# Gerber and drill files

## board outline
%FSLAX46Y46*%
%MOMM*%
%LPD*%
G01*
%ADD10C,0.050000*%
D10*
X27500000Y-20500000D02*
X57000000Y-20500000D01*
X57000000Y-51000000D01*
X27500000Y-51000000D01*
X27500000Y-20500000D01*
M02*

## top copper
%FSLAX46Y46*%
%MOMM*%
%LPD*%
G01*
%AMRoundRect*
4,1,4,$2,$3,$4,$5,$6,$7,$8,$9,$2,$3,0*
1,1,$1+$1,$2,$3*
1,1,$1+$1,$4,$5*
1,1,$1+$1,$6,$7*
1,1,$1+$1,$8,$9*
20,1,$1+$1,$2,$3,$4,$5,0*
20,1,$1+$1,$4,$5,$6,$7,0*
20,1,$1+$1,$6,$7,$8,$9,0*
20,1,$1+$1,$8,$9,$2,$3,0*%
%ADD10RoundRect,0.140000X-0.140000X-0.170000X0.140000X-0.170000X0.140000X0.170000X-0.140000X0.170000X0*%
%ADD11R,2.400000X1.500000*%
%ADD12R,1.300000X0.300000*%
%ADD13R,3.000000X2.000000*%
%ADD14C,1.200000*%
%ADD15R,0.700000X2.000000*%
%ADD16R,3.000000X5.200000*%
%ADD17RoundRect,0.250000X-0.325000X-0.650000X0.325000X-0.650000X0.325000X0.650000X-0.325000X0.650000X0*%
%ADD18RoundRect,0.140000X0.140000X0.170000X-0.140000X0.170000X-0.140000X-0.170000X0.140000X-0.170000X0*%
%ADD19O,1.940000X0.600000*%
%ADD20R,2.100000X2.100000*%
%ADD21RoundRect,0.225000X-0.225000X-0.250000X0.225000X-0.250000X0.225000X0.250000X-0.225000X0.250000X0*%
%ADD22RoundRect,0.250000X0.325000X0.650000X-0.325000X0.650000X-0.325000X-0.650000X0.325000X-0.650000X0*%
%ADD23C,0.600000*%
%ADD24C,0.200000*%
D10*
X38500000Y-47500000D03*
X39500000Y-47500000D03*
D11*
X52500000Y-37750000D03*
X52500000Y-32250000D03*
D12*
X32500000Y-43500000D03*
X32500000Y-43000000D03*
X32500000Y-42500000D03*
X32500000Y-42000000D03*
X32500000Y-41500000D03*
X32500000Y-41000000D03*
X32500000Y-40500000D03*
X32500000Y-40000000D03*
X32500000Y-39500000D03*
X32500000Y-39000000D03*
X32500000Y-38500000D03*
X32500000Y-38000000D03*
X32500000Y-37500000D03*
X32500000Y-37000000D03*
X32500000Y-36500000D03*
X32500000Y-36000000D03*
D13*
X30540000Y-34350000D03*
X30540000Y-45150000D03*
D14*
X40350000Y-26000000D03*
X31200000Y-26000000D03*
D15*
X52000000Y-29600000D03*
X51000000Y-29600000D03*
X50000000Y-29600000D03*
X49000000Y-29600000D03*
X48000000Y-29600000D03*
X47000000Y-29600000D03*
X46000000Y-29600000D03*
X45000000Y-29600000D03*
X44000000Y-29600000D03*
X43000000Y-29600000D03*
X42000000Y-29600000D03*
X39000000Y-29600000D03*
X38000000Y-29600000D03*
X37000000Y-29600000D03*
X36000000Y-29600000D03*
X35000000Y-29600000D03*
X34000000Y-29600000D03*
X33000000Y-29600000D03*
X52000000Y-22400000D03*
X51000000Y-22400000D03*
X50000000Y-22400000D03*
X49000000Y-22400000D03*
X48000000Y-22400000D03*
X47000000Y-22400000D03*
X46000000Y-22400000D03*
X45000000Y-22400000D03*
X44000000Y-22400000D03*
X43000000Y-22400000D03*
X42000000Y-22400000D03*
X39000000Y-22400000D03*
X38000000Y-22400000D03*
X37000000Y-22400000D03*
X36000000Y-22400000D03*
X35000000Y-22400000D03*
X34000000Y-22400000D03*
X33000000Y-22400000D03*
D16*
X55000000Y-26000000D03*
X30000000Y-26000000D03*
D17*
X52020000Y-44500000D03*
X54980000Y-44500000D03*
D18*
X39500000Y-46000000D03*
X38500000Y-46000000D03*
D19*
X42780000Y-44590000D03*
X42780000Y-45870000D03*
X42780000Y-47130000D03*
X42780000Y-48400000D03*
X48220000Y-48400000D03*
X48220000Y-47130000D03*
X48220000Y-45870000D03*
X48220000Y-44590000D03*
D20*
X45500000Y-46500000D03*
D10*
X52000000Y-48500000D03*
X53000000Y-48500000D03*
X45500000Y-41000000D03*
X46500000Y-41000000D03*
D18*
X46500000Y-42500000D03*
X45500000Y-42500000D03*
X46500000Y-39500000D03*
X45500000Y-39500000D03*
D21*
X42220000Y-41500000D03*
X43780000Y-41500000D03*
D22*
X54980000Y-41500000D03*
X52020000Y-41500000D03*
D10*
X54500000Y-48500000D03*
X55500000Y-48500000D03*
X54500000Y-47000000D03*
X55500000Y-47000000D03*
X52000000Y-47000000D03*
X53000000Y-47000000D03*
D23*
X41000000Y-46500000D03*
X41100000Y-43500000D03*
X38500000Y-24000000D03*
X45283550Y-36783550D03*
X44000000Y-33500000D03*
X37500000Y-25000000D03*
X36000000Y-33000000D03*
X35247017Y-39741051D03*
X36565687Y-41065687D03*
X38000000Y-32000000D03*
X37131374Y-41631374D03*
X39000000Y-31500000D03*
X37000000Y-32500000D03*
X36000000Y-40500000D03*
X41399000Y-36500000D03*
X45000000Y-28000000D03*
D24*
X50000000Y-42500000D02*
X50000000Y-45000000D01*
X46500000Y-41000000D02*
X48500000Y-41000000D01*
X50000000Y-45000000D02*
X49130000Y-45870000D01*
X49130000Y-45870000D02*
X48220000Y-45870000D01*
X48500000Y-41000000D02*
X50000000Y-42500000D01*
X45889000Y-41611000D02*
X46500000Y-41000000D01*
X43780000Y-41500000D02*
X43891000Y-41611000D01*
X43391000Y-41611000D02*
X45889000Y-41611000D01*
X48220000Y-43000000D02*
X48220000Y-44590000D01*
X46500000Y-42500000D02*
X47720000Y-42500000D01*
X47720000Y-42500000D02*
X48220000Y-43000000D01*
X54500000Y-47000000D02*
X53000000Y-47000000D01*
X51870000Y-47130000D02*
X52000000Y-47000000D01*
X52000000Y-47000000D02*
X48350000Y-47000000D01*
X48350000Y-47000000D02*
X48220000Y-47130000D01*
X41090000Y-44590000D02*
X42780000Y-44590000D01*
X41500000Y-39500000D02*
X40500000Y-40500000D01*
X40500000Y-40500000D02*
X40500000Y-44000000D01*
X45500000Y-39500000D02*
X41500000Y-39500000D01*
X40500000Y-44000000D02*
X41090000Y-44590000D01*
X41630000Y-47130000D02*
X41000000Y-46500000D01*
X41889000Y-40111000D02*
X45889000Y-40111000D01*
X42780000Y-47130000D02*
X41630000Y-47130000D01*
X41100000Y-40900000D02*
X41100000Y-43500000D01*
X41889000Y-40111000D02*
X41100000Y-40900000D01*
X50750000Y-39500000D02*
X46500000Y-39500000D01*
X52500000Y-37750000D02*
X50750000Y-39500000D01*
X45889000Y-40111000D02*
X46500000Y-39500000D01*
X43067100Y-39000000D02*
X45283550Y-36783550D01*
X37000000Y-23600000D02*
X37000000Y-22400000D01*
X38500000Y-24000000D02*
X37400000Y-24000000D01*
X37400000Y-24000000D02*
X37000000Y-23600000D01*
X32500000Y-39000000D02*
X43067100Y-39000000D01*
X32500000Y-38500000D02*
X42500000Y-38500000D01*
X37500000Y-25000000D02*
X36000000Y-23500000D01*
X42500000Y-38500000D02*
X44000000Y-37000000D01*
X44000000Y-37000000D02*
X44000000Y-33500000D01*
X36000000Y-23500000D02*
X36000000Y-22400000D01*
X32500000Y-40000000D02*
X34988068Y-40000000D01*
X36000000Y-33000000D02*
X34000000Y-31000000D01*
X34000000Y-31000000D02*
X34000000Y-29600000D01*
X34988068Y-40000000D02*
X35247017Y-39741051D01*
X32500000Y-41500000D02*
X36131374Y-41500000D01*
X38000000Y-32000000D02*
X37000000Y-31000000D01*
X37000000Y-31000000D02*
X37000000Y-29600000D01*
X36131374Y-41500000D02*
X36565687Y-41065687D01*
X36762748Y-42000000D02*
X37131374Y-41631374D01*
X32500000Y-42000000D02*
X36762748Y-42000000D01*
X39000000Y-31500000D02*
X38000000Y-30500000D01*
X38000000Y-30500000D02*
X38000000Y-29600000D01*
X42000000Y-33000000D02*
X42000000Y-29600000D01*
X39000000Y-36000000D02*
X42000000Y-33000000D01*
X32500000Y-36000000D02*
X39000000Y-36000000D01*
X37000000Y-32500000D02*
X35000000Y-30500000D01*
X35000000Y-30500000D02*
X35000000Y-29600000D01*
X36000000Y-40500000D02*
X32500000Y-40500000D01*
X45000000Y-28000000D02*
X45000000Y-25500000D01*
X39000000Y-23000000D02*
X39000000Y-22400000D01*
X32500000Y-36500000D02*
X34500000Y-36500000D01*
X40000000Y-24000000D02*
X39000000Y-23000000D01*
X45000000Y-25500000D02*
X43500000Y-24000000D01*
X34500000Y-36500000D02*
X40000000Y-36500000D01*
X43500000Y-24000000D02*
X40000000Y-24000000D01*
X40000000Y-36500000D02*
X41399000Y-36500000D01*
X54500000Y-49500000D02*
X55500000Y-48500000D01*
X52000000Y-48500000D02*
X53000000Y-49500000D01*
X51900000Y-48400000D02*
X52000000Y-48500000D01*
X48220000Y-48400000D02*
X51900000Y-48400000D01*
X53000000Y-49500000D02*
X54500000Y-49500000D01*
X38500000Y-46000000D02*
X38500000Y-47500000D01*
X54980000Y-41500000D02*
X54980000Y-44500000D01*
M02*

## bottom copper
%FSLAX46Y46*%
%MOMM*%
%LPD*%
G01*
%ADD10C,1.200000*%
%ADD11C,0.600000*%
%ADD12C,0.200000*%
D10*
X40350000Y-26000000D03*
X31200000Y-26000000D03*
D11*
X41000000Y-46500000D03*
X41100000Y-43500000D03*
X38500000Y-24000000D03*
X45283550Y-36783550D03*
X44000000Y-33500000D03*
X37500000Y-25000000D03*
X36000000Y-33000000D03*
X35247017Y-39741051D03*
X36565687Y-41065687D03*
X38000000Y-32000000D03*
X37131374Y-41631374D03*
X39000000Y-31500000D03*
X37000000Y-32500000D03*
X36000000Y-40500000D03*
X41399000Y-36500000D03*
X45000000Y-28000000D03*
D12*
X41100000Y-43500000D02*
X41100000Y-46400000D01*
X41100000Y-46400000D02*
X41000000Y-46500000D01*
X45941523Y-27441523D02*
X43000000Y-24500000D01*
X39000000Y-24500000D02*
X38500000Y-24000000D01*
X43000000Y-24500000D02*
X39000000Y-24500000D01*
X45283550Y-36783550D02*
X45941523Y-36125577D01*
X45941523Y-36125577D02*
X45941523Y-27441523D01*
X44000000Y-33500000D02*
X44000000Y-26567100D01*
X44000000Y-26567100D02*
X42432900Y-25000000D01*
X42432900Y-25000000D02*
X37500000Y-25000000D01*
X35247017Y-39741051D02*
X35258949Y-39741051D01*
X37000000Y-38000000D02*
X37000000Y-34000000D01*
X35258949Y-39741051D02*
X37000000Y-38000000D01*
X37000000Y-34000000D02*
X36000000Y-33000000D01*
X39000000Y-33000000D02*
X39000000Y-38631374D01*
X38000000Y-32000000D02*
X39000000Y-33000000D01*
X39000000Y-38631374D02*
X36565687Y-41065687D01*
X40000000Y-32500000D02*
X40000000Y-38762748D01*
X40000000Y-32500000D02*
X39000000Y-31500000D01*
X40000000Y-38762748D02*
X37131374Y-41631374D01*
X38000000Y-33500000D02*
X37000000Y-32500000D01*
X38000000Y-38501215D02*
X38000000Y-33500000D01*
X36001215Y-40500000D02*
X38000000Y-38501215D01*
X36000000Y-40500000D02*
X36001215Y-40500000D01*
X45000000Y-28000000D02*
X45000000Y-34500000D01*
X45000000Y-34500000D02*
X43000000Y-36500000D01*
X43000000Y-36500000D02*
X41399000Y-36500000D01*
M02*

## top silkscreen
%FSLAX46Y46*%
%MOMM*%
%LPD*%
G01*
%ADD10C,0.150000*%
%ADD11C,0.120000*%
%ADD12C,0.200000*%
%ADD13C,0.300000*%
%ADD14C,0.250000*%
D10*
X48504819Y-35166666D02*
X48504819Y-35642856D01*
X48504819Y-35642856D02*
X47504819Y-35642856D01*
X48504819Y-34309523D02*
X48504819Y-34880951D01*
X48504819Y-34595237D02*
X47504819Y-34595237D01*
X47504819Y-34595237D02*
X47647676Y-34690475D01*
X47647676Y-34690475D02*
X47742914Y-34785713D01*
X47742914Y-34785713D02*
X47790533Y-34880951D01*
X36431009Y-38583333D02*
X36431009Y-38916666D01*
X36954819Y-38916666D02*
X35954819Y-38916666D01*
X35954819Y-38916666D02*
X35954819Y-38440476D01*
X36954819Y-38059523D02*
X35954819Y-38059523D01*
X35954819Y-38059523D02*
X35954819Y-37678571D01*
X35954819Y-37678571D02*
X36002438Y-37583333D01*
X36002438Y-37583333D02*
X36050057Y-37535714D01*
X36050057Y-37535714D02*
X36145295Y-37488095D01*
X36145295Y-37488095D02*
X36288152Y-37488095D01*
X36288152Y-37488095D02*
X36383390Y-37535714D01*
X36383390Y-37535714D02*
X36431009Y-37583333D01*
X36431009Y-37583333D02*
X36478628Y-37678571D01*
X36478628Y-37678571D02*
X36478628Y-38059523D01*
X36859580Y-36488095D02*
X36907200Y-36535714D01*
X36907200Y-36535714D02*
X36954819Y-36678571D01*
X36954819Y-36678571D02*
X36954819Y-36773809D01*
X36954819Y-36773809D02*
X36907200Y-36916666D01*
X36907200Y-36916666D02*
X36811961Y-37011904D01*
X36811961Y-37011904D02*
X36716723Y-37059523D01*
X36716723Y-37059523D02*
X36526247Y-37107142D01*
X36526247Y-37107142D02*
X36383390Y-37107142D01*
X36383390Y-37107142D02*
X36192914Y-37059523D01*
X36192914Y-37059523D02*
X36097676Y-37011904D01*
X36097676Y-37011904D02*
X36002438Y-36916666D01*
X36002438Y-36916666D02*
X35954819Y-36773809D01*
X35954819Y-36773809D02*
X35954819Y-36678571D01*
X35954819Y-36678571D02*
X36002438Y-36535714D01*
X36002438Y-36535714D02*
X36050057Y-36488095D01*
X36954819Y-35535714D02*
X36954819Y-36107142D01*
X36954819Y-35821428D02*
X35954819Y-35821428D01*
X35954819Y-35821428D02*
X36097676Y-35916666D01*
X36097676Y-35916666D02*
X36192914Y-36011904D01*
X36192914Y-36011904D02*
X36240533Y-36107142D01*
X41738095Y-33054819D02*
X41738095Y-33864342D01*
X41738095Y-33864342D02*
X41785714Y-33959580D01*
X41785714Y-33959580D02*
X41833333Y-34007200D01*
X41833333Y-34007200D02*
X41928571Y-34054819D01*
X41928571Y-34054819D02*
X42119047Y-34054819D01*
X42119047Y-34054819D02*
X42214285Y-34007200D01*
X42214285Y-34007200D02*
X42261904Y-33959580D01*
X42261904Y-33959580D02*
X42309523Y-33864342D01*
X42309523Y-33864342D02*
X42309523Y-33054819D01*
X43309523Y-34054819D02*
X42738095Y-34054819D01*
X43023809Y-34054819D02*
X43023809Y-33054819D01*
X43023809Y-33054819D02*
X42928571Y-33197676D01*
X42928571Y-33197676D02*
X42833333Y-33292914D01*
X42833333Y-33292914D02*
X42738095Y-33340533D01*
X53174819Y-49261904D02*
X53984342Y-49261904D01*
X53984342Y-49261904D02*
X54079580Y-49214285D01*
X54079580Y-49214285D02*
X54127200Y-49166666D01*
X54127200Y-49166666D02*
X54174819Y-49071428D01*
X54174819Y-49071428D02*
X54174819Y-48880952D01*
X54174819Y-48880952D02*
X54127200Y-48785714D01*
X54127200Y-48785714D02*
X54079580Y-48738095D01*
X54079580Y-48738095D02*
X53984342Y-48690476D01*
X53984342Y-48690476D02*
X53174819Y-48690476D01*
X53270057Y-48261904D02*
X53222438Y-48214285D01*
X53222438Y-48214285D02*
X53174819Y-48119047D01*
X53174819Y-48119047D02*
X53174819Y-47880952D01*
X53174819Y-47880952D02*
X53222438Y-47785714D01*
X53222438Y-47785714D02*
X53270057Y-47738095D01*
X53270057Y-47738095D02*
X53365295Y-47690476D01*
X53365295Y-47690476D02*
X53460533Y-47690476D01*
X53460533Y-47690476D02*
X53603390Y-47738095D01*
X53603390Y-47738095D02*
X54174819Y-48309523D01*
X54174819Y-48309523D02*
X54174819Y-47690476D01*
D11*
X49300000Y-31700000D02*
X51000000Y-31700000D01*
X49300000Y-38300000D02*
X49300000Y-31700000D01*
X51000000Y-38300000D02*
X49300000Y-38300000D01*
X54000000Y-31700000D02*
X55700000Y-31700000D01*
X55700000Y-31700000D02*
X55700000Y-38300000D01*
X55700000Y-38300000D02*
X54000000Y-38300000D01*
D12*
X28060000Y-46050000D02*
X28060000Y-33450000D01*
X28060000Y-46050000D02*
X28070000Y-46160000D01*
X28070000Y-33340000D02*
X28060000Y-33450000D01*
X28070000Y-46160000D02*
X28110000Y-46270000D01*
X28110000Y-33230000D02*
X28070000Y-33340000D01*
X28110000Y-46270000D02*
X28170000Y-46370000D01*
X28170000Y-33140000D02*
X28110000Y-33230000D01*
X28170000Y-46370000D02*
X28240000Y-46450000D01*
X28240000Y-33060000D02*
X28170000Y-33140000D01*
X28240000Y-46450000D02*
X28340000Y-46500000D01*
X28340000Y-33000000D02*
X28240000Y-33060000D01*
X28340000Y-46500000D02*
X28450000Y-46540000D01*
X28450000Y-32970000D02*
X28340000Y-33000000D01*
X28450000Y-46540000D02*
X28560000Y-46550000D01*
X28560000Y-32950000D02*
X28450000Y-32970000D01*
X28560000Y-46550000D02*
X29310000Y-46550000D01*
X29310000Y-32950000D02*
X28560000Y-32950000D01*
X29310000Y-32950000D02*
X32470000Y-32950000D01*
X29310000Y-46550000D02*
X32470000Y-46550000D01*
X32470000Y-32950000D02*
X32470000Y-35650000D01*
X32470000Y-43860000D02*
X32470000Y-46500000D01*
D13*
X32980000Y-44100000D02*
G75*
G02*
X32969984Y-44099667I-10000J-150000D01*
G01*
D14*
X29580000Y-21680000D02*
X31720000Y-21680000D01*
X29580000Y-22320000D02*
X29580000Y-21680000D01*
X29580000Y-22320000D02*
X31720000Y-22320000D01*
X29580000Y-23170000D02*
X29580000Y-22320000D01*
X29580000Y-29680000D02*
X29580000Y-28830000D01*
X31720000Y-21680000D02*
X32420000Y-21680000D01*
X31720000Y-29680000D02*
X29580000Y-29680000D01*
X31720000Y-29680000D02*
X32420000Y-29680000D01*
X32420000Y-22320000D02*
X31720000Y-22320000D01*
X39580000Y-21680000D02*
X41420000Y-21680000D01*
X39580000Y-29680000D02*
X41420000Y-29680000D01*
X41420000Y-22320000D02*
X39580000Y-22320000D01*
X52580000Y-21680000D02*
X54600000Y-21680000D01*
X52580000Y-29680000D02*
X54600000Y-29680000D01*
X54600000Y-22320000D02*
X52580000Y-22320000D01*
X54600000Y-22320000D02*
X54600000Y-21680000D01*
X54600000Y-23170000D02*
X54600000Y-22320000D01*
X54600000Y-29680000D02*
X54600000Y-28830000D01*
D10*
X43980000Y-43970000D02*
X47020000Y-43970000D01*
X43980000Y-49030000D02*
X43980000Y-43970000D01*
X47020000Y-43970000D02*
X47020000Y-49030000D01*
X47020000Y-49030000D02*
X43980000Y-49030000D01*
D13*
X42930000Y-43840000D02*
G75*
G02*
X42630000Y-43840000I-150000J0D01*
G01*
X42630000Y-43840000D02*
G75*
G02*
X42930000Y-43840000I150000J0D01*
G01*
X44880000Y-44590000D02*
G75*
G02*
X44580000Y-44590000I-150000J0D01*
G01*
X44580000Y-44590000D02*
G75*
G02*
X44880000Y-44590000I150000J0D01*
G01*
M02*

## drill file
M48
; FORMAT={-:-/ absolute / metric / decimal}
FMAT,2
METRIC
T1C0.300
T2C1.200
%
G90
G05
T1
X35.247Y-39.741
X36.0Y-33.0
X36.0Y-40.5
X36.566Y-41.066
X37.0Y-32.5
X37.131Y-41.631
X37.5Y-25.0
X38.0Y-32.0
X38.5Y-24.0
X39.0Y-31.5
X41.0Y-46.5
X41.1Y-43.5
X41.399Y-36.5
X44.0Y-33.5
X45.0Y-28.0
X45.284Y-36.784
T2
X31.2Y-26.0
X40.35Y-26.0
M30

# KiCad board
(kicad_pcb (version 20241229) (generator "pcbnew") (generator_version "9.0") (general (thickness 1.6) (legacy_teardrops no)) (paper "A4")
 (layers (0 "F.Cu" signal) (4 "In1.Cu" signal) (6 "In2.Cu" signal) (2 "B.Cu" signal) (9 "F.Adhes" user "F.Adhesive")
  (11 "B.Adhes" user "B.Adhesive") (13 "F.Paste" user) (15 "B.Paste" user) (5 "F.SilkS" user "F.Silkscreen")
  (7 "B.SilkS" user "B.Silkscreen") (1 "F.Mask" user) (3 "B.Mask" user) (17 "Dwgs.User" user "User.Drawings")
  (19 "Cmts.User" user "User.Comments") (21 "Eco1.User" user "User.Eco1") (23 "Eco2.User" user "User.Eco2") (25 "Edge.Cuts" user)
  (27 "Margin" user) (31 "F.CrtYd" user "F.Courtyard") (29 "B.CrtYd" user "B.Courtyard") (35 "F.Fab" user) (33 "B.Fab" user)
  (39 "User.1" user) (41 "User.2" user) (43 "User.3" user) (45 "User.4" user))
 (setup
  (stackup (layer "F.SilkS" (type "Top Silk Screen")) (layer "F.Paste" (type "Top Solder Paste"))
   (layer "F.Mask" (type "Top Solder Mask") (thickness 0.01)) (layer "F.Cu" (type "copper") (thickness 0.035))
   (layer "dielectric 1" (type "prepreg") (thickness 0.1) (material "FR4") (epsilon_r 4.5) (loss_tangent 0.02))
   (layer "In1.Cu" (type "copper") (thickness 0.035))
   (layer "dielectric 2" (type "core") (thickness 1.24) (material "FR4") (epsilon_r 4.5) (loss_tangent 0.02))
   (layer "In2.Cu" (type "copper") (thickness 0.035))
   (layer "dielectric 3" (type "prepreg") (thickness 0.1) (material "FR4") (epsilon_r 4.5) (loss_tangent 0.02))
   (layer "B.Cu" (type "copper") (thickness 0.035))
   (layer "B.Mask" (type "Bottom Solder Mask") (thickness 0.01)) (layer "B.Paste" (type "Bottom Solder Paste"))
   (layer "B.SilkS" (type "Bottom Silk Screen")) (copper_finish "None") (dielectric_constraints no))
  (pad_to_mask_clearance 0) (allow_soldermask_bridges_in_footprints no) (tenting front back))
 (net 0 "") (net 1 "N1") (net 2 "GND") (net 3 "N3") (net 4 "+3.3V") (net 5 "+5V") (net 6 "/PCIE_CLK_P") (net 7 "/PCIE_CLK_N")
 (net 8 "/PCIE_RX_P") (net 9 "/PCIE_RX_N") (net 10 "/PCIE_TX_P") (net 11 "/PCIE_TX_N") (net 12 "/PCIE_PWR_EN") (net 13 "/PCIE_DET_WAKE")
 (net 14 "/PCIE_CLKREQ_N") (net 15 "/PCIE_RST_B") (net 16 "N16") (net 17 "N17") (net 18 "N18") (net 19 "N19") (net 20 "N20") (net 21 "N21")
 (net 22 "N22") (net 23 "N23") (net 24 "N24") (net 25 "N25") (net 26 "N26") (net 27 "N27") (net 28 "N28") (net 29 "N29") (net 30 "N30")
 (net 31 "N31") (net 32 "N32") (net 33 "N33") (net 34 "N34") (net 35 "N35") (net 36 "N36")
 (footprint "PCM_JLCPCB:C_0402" (layer "F.Cu") (at 39 47.5)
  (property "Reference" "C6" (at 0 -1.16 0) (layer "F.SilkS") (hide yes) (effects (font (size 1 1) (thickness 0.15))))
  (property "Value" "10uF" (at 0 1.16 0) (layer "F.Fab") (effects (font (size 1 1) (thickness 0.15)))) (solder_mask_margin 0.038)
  (pad "1" smd roundrect (at -0.5 0) (size 0.56 0.62) (layers "F.Cu" "F.Mask" "F.Paste") (roundrect_rratio 0.25) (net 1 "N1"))
  (pad "2" smd roundrect (at 0.5 0) (size 0.56 0.62) (layers "F.Cu" "F.Mask" "F.Paste") (roundrect_rratio 0.25) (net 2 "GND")))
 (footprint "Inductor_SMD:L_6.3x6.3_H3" (layer "F.Cu") (at 52.5 35 90)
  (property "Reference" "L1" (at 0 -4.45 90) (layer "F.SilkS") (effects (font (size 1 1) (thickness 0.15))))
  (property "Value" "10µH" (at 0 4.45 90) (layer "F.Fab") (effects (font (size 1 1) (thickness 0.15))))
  (fp_line (start 3.3 -3.2) (end 3.3 -1.5) (stroke (width 0.12) (type solid)) (layer "F.SilkS"))
  (fp_line (start -3.3 -3.2) (end 3.3 -3.2) (stroke (width 0.12) (type solid)) (layer "F.SilkS"))
  (fp_line (start -3.3 -1.5) (end -3.3 -3.2) (stroke (width 0.12) (type solid)) (layer "F.SilkS"))
  (fp_line (start 3.3 1.5) (end 3.3 3.2) (stroke (width 0.12) (type solid)) (layer "F.SilkS"))
  (fp_line (start 3.3 3.2) (end -3.3 3.2) (stroke (width 0.12) (type solid)) (layer "F.SilkS"))
  (fp_line (start -3.3 3.2) (end -3.3 1.5) (stroke (width 0.12) (type solid)) (layer "F.SilkS"))
  (pad "1" smd rect (at -2.75 0 90) (size 1.5 2.4) (layers "F.Cu" "F.Mask" "F.Paste") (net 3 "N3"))
  (pad "2" smd rect (at 2.75 0 90) (size 1.5 2.4) (layers "F.Cu" "F.Mask" "F.Paste") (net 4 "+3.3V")))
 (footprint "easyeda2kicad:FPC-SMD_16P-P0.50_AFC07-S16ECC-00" (layer "F.Cu") (at 31.52 39.75 -90)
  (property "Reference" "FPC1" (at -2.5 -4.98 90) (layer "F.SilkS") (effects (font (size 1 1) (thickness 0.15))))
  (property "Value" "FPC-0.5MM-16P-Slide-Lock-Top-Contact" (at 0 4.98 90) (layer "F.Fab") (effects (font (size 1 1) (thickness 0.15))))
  (fp_line (start 6.3 3.46) (end -6.3 3.46) (stroke (width 0.2) (type solid)) (layer "F.SilkS"))
  (fp_line (start 6.3 3.46) (end 6.41 3.45) (stroke (width 0.2) (type solid)) (layer "F.SilkS"))
  (fp_line (start -6.41 3.45) (end -6.3 3.46) (stroke (width 0.2) (type solid)) (layer "F.SilkS"))
  (fp_line (start 6.41 3.45) (end 6.52 3.41) (stroke (width 0.2) (type solid)) (layer "F.SilkS"))
  (fp_line (start -6.52 3.41) (end -6.41 3.45) (stroke (width 0.2) (type solid)) (layer "F.SilkS"))
  (fp_line (start 6.52 3.41) (end 6.62 3.35) (stroke (width 0.2) (type solid)) (layer "F.SilkS"))
  (fp_line (start -6.61 3.35) (end -6.52 3.41) (stroke (width 0.2) (type solid)) (layer "F.SilkS"))
  (fp_line (start 6.62 3.35) (end 6.7 3.28) (stroke (width 0.2) (type solid)) (layer "F.SilkS"))
  (fp_line (start -6.69 3.28) (end -6.61 3.35) (stroke (width 0.2) (type solid)) (layer "F.SilkS"))
  (fp_line (start 6.7 3.28) (end 6.75 3.18) (stroke (width 0.2) (type solid)) (layer "F.SilkS"))
  (fp_line (start -6.75 3.18) (end -6.69 3.28) (stroke (width 0.2) (type solid)) (layer "F.SilkS"))
  (fp_line (start 6.75 3.18) (end 6.79 3.07) (stroke (width 0.2) (type solid)) (layer "F.SilkS"))
  (fp_line (start -6.78 3.07) (end -6.75 3.18) (stroke (width 0.2) (type solid)) (layer "F.SilkS"))
  (fp_line (start 6.79 3.07) (end 6.8 2.96) (stroke (width 0.2) (type solid)) (layer "F.SilkS"))
  (fp_line (start -6.8 2.96) (end -6.78 3.07) (stroke (width 0.2) (type solid)) (layer "F.SilkS"))
  (fp_line (start 6.8 2.96) (end 6.8 2.21) (stroke (width 0.2) (type solid)) (layer "F.SilkS"))
  (fp_line (start -6.8 2.21) (end -6.8 2.96) (stroke (width 0.2) (type solid)) (layer "F.SilkS"))
  (fp_line (start -6.8 2.21) (end -6.8 -0.95) (stroke (width 0.2) (type solid)) (layer "F.SilkS"))
  (fp_line (start 6.8 2.21) (end 6.8 -0.95) (stroke (width 0.2) (type solid)) (layer "F.SilkS"))
  (fp_line (start -6.8 -0.95) (end -4.1 -0.95) (stroke (width 0.2) (type solid)) (layer "F.SilkS"))
  (fp_line (start 4.11 -0.95) (end 6.75 -0.95) (stroke (width 0.2) (type solid)) (layer "F.SilkS"))
  (fp_arc (start 4.35 -1.46) (mid 4.65025 -1.445005) (end 4.349667 -1.449984) (stroke (width 0.3) (type solid)) (layer "F.SilkS"))
  (pad "1" smd rect (at 3.75 -0.98 90) (size 0.3 1.3) (layers "F.Cu" "F.Mask" "F.Paste") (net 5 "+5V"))
  (pad "2" smd rect (at 3.25 -0.98 90) (size 0.3 1.3) (layers "F.Cu" "F.Mask" "F.Paste") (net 5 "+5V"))
  (pad "3" smd rect (at 2.75 -0.98 90) (size 0.3 1.3) (layers "F.Cu" "F.Mask" "F.Paste") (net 2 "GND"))
  (pad "4" smd rect (at 2.25 -0.98 90) (size 0.3 1.3) (layers "F.Cu" "F.Mask" "F.Paste") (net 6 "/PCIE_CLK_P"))
  (pad "5" smd rect (at 1.75 -0.98 90) (size 0.3 1.3) (layers "F.Cu" "F.Mask" "F.Paste") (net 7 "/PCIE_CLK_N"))
  (pad "6" smd rect (at 1.25 -0.98 90) (size 0.3 1.3) (layers "F.Cu" "F.Mask" "F.Paste") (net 2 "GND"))
  (pad "7" smd rect (at 0.75 -0.98 90) (size 0.3 1.3) (layers "F.Cu" "F.Mask" "F.Paste") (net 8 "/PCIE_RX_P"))
  (pad "8" smd rect (at 0.25 -0.98 90) (size 0.3 1.3) (layers "F.Cu" "F.Mask" "F.Paste") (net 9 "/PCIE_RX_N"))
  (pad "9" smd rect (at -0.25 -0.98 90) (size 0.3 1.3) (layers "F.Cu" "F.Mask" "F.Paste") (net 2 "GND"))
  (pad "10" smd rect (at -0.75 -0.98 90) (size 0.3 1.3) (layers "F.Cu" "F.Mask" "F.Paste") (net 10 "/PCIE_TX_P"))
  (pad "11" smd rect (at -1.25 -0.98 90) (size 0.3 1.3) (layers "F.Cu" "F.Mask" "F.Paste") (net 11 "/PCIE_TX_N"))
  (pad "12" smd rect (at -1.75 -0.98 90) (size 0.3 1.3) (layers "F.Cu" "F.Mask" "F.Paste") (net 2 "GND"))
  (pad "13" smd rect (at -2.25 -0.98 90) (size 0.3 1.3) (layers "F.Cu" "F.Mask" "F.Paste") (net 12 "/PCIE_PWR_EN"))
  (pad "14" smd rect (at -2.75 -0.98 90) (size 0.3 1.3) (layers "F.Cu" "F.Mask" "F.Paste") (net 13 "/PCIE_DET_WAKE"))
  (pad "15" smd rect (at -3.25 -0.98 90) (size 0.3 1.3) (layers "F.Cu" "F.Mask" "F.Paste") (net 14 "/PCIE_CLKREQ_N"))
  (pad "16" smd rect (at -3.75 -0.98 90) (size 0.3 1.3) (layers "F.Cu" "F.Mask" "F.Paste") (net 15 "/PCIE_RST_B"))
  (pad "17" smd rect (at -5.4 0.98 270) (size 2 3) (layers "F.Cu" "F.Mask" "F.Paste") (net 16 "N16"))
  (pad "18" smd rect (at 5.4 0.98 90) (size 2 3) (layers "F.Cu" "F.Mask" "F.Paste") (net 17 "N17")))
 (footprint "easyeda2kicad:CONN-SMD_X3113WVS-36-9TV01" (layer "F.Cu") (at 42.5 26 180)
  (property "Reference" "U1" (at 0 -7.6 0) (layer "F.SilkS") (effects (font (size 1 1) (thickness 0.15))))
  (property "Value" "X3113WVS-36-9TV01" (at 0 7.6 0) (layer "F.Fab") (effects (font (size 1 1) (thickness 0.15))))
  (fp_line (start 12.92 4.32) (end 10.78 4.32) (stroke (width 0.25) (type solid)) (layer "F.SilkS"))
  (fp_line (start 12.92 3.68) (end 12.92 4.32) (stroke (width 0.25) (type solid)) (layer "F.SilkS"))
  (fp_line (start 12.92 3.68) (end 10.78 3.68) (stroke (width 0.25) (type solid)) (layer "F.SilkS"))
  (fp_line (start 12.92 2.83) (end 12.92 3.68) (stroke (width 0.25) (type solid)) (layer "F.SilkS"))
  (fp_line (start 12.92 -3.68) (end 12.92 -2.83) (stroke (width 0.25) (type solid)) (layer "F.SilkS"))
  (fp_line (start 10.78 4.32) (end 10.08 4.32) (stroke (width 0.25) (type solid)) (layer "F.SilkS"))
  (fp_line (start 10.78 -3.68) (end 12.92 -3.68) (stroke (width 0.25) (type solid)) (layer "F.SilkS"))
  (fp_line (start 10.78 -3.68) (end 10.08 -3.68) (stroke (width 0.25) (type solid)) (layer "F.SilkS"))
  (fp_line (start 10.08 3.68) (end 10.78 3.68) (stroke (width 0.25) (type solid)) (layer "F.SilkS"))
  (fp_line (start 2.92 4.32) (end 1.08 4.32) (stroke (width 0.25) (type solid)) (layer "F.SilkS"))
  (fp_line (start 2.92 -3.68) (end 1.08 -3.68) (stroke (width 0.25) (type solid)) (layer "F.SilkS"))
  (fp_line (start 1.08 3.68) (end 2.92 3.68) (stroke (width 0.25) (type solid)) (layer "F.SilkS"))
  (fp_line (start -10.08 4.32) (end -12.1 4.32) (stroke (width 0.25) (type solid)) (layer "F.SilkS"))
  (fp_line (start -10.08 -3.68) (end -12.1 -3.68) (stroke (width 0.25) (type solid)) (layer "F.SilkS"))
  (fp_line (start -12.1 3.68) (end -10.08 3.68) (stroke (width 0.25) (type solid)) (layer "F.SilkS"))
  (fp_line (start -12.1 3.68) (end -12.1 4.32) (stroke (width 0.25) (type solid)) (layer "F.SilkS"))
  (fp_line (start -12.1 2.83) (end -12.1 3.68) (stroke (width 0.25) (type solid)) (layer "F.SilkS"))
  (fp_line (start -12.1 -3.68) (end -12.1 -2.83) (stroke (width 0.25) (type solid)) (layer "F.SilkS"))
  (pad "" thru_hole circle (at 2.15 0 180) (size 1.2 1.2) (drill 1.2) (layers "*.Cu" "*.Mask") (remove_unused_layers no))
  (pad "" thru_hole circle (at 11.3 0 180) (size 1.2 1.2) (drill 1.2) (layers "*.Cu" "*.Mask") (remove_unused_layers no))
  (pad "1" smd rect (at -9.5 -3.6 180) (size 0.7 2) (layers "F.Cu" "F.Mask" "F.Paste") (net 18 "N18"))
  (pad "2" smd rect (at -8.5 -3.6 180) (size 0.7 2) (layers "F.Cu" "F.Mask" "F.Paste") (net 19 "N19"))
  (pad "3" smd rect (at -7.5 -3.6 180) (size 0.7 2) (layers "F.Cu" "F.Mask" "F.Paste") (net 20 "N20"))
  (pad "4" smd rect (at -6.5 -3.6 180) (size 0.7 2) (layers "F.Cu" "F.Mask" "F.Paste") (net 2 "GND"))
  (pad "5" smd rect (at -5.5 -3.6 180) (size 0.7 2) (layers "F.Cu" "F.Mask" "F.Paste") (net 4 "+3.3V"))
  (pad "6" smd rect (at -4.5 -3.6 180) (size 0.7 2) (layers "F.Cu" "F.Mask" "F.Paste") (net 4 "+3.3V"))
  (pad "7" smd rect (at -3.5 -3.6 180) (size 0.7 2) (layers "F.Cu" "F.Mask" "F.Paste") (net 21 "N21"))
  (pad "8" smd rect (at -2.5 -3.6 180) (size 0.7 2) (layers "F.Cu" "F.Mask" "F.Paste") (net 4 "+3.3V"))
  (pad "9" smd rect (at -1.5 -3.6 180) (size 0.7 2) (layers "F.Cu" "F.Mask" "F.Paste") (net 4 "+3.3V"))
  (pad "10" smd rect (at -0.5 -3.6 180) (size 0.7 2) (layers "F.Cu" "F.Mask" "F.Paste") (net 4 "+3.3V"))
  (pad "11" smd rect (at 0.5 -3.6 180) (size 0.7 2) (layers "F.Cu" "F.Mask" "F.Paste") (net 15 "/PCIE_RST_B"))
  (pad "12" smd rect (at 3.5 -3.6 180) (size 0.7 2) (layers "F.Cu" "F.Mask" "F.Paste") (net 2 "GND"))
  (pad "13" smd rect (at 4.5 -3.6 180) (size 0.7 2) (layers "F.Cu" "F.Mask" "F.Paste") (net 6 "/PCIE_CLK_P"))
  (pad "14" smd rect (at 5.5 -3.6 180) (size 0.7 2) (layers "F.Cu" "F.Mask" "F.Paste") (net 7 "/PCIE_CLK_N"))
  (pad "15" smd rect (at 6.5 -3.6 180) (size 0.7 2) (layers "F.Cu" "F.Mask" "F.Paste") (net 2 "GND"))
  (pad "16" smd rect (at 7.5 -3.6 180) (size 0.7 2) (layers "F.Cu" "F.Mask" "F.Paste") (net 8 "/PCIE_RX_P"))
  (pad "17" smd rect (at 8.5 -3.6 180) (size 0.7 2) (layers "F.Cu" "F.Mask" "F.Paste") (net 9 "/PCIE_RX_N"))
  (pad "18" smd rect (at 9.5 -3.6 180) (size 0.7 2) (layers "F.Cu" "F.Mask" "F.Paste") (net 2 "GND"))
  (pad "19" smd rect (at -9.5 3.6 180) (size 0.7 2) (layers "F.Cu" "F.Mask" "F.Paste") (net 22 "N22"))
  (pad "20" smd rect (at -8.5 3.6 180) (size 0.7 2) (layers "F.Cu" "F.Mask" "F.Paste") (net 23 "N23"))
  (pad "21" smd rect (at -7.5 3.6 180) (size 0.7 2) (layers "F.Cu" "F.Mask" "F.Paste") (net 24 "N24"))
  (pad "22" smd rect (at -6.5 3.6 180) (size 0.7 2) (layers "F.Cu" "F.Mask" "F.Paste") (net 2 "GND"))
  (pad "23" smd rect (at -5.5 3.6 180) (size 0.7 2) (layers "F.Cu" "F.Mask" "F.Paste") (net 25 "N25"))
  (pad "24" smd rect (at -4.5 3.6 180) (size 0.7 2) (layers "F.Cu" "F.Mask" "F.Paste") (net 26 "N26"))
  (pad "25" smd rect (at -3.5 3.6 180) (size 0.7 2) (layers "F.Cu" "F.Mask" "F.Paste") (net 2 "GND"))
  (pad "26" smd rect (at -2.5 3.6 180) (size 0.7 2) (layers "F.Cu" "F.Mask" "F.Paste") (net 4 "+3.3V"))
  (pad "27" smd rect (at -1.5 3.6 180) (size 0.7 2) (layers "F.Cu" "F.Mask" "F.Paste") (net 4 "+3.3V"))
  (pad "28" smd rect (at -0.5 3.6 180) (size 0.7 2) (layers "F.Cu" "F.Mask" "F.Paste") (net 4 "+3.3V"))
  (pad "29" smd rect (at 0.5 3.6 180) (size 0.7 2) (layers "F.Cu" "F.Mask" "F.Paste") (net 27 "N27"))
  (pad "30" smd rect (at 3.5 3.6 180) (size 0.7 2) (layers "F.Cu" "F.Mask" "F.Paste") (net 14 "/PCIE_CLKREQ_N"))
  (pad "31" smd rect (at 4.5 3.6 180) (size 0.7 2) (layers "F.Cu" "F.Mask" "F.Paste") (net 2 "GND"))
  (pad "32" smd rect (at 5.5 3.6 180) (size 0.7 2) (layers "F.Cu" "F.Mask" "F.Paste") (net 10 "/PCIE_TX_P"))
  (pad "33" smd rect (at 6.5 3.6 180) (size 0.7 2) (layers "F.Cu" "F.Mask" "F.Paste") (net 11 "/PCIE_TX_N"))
  (pad "34" smd rect (at 7.5 3.6 180) (size 0.7 2) (layers "F.Cu" "F.Mask" "F.Paste") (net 2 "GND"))
  (pad "35" smd rect (at 8.5 3.6 180) (size 0.7 2) (layers "F.Cu" "F.Mask" "F.Paste") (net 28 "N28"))
  (pad "36" smd rect (at 9.5 3.6 180) (size 0.7 2) (layers "F.Cu" "F.Mask" "F.Paste") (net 2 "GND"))
  (pad "37" smd rect (at -12.5 0 180) (size 3 5.2) (layers "F.Cu" "F.Mask" "F.Paste") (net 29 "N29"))
  (pad "37" smd rect (at 12.5 0 180) (size 3 5.2) (layers "F.Cu" "F.Mask" "F.Paste") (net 29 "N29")))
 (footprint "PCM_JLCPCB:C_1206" (layer "F.Cu") (at 53.5 44.5)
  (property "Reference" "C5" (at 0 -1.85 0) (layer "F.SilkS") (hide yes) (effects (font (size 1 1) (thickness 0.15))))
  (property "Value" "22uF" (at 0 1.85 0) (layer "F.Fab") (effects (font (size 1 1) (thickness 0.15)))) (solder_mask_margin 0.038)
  (pad "1" smd roundrect (at -1.48 0) (size 1.15 1.8) (layers "F.Cu" "F.Mask" "F.Paste") (roundrect_rratio 0.217391) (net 4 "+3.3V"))
  (pad "2" smd roundrect (at 1.48 0) (size 1.15 1.8) (layers "F.Cu" "F.Mask" "F.Paste") (roundrect_rratio 0.217391) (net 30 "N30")))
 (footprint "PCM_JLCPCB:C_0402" (layer "F.Cu") (at 39 46 180)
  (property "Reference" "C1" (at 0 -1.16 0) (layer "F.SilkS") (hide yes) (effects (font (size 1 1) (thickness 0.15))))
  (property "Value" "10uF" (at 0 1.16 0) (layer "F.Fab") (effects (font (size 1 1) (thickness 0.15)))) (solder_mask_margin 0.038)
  (pad "1" smd roundrect (at -0.5 0 180) (size 0.56 0.62) (layers "F.Cu" "F.Mask" "F.Paste") (roundrect_rratio 0.25) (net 5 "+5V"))
  (pad "2" smd roundrect (at 0.5 0 180) (size 0.56 0.62) (layers "F.Cu" "F.Mask" "F.Paste") (roundrect_rratio 0.25) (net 1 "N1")))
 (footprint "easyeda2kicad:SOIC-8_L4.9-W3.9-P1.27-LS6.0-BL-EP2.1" (layer "F.Cu") (at 45.5 46.5 -90)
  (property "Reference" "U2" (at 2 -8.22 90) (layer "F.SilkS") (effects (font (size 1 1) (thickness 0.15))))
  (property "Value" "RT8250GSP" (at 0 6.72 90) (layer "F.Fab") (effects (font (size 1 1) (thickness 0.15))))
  (fp_line (start -2.53 1.52) (end -2.53 -1.52) (stroke (width 0.15) (type solid)) (layer "F.SilkS"))
  (fp_line (start 2.53 1.52) (end -2.53 1.52) (stroke (width 0.15) (type solid)) (layer "F.SilkS"))
  (fp_line (start -2.53 -1.52) (end 2.53 -1.52) (stroke (width 0.15) (type solid)) (layer "F.SilkS"))
  (fp_line (start 2.53 -1.52) (end 2.53 1.52) (stroke (width 0.15) (type solid)) (layer "F.SilkS"))
  (fp_circle (center -2.66 2.72) (end -2.51 2.72) (stroke (width 0.3) (type solid)) (fill no) (layer "F.SilkS"))
  (fp_circle (center -1.91 0.77) (end -1.76 0.77) (stroke (width 0.3) (type solid)) (fill no) (layer "F.SilkS"))
  (pad "1" smd oval (at -1.91 2.72 270) (size 0.6 1.94) (layers "F.Cu" "F.Mask" "F.Paste") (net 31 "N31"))
  (pad "2" smd oval (at -0.63 2.72 270) (size 0.6 1.94) (layers "F.Cu" "F.Mask" "F.Paste") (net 5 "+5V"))
  (pad "3" smd oval (at 0.63 2.72 270) (size 0.6 1.94) (layers "F.Cu" "F.Mask" "F.Paste") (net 3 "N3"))
  (pad "4" smd oval (at 1.9 2.72 270) (size 0.6 1.94) (layers "F.Cu" "F.Mask" "F.Paste") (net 2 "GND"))
  (pad "5" smd oval (at 1.9 -2.72 270) (size 0.6 1.94) (layers "F.Cu" "F.Mask" "F.Paste") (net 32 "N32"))
  (pad "6" smd oval (at 0.63 -2.72 270) (size 0.6 1.94) (layers "F.Cu" "F.Mask" "F.Paste") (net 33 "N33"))
  (pad "7" smd oval (at -0.63 -2.72 270) (size 0.6 1.94) (layers "F.Cu" "F.Mask" "F.Paste") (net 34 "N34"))
  (pad "8" smd oval (at -1.91 -2.72 270) (size 0.6 1.94) (layers "F.Cu" "F.Mask" "F.Paste") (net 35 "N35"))
  (pad "9" smd rect (at 0 0 270) (size 2.1 2.1) (layers "F.Cu" "F.Mask" "F.Paste") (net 2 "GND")))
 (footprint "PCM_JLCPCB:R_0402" (layer "F.Cu") (at 52.5 48.5)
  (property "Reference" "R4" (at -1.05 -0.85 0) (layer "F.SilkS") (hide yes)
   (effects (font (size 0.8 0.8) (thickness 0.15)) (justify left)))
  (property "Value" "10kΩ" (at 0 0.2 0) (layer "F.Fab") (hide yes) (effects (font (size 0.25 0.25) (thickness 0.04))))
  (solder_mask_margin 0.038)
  (pad "1" smd roundrect (at -0.5 0) (size 0.56 0.62) (layers "F.Cu" "F.Mask" "F.Paste") (roundrect_rratio 0.25) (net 32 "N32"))
  (pad "2" smd roundrect (at 0.5 0) (size 0.56 0.62) (layers "F.Cu" "F.Mask" "F.Paste") (roundrect_rratio 0.25) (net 2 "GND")))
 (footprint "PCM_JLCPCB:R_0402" (layer "F.Cu") (at 46 41)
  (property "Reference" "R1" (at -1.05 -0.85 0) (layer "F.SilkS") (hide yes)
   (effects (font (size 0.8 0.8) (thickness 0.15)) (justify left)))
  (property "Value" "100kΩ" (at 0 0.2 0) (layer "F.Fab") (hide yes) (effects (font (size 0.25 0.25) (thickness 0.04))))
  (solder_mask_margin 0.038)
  (pad "1" smd roundrect (at -0.5 0) (size 0.56 0.62) (layers "F.Cu" "F.Mask" "F.Paste") (roundrect_rratio 0.25) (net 5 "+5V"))
  (pad "2" smd roundrect (at 0.5 0) (size 0.56 0.62) (layers "F.Cu" "F.Mask" "F.Paste") (roundrect_rratio 0.25) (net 34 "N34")))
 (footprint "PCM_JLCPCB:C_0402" (layer "F.Cu") (at 46 42.5 180)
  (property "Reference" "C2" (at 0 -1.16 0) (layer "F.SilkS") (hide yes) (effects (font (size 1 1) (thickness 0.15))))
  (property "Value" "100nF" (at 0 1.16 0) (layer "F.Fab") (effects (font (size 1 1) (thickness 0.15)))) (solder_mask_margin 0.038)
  (pad "1" smd roundrect (at -0.5 0 180) (size 0.56 0.62) (layers "F.Cu" "F.Mask" "F.Paste") (roundrect_rratio 0.25) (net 35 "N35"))
  (pad "2" smd roundrect (at 0.5 0 180) (size 0.56 0.62) (layers "F.Cu" "F.Mask" "F.Paste") (roundrect_rratio 0.25) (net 2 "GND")))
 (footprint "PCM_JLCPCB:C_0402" (layer "F.Cu") (at 46 39.5 180)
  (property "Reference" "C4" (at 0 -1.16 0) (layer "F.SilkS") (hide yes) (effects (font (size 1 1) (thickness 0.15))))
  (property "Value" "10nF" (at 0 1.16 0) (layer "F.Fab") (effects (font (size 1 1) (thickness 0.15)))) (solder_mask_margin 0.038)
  (pad "1" smd roundrect (at -0.5 0 180) (size 0.56 0.62) (layers "F.Cu" "F.Mask" "F.Paste") (roundrect_rratio 0.25) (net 3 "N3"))
  (pad "2" smd roundrect (at 0.5 0 180) (size 0.56 0.62) (layers "F.Cu" "F.Mask" "F.Paste") (roundrect_rratio 0.25) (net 31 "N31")))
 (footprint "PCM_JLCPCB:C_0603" (layer "F.Cu") (at 43 41.5)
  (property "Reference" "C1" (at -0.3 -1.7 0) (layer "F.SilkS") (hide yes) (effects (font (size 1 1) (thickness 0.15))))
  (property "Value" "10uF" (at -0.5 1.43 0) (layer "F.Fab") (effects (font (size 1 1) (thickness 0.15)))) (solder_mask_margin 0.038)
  (pad "1" smd roundrect (at -0.78 0) (size 0.9 0.95) (layers "F.Cu" "F.Mask" "F.Paste") (roundrect_rratio 0.25) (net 5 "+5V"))
  (pad "2" smd roundrect (at 0.78 0) (size 0.9 0.95) (layers "F.Cu" "F.Mask" "F.Paste") (roundrect_rratio 0.25) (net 34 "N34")))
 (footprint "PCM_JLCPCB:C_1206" (layer "F.Cu") (at 53.5 41.5 180)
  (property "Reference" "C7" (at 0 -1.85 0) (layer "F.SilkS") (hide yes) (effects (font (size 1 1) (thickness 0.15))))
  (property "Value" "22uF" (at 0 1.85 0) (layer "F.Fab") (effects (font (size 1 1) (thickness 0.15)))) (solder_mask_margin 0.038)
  (pad "1" smd roundrect (at -1.48 0 180) (size 1.15 1.8) (layers "F.Cu" "F.Mask" "F.Paste") (roundrect_rratio 0.217391) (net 30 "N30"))
  (pad "2" smd roundrect (at 1.48 0 180) (size 1.15 1.8) (layers "F.Cu" "F.Mask" "F.Paste") (roundrect_rratio 0.217391) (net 2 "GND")))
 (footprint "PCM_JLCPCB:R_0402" (layer "F.Cu") (at 55 48.5)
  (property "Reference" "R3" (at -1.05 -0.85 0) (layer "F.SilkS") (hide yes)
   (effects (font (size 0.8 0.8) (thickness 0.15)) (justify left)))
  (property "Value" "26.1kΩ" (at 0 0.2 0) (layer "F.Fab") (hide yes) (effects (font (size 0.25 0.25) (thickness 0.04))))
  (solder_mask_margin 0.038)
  (pad "1" smd roundrect (at -0.5 0) (size 0.56 0.62) (layers "F.Cu" "F.Mask" "F.Paste") (roundrect_rratio 0.25) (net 4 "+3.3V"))
  (pad "2" smd roundrect (at 0.5 0) (size 0.56 0.62) (layers "F.Cu" "F.Mask" "F.Paste") (roundrect_rratio 0.25) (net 32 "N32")))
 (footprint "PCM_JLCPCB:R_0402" (layer "F.Cu") (at 55 47)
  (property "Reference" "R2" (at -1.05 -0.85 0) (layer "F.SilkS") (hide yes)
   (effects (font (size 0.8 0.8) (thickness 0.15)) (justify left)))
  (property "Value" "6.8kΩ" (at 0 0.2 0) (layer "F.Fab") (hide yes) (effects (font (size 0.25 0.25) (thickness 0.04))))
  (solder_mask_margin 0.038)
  (pad "1" smd roundrect (at -0.5 0) (size 0.56 0.62) (layers "F.Cu" "F.Mask" "F.Paste") (roundrect_rratio 0.25) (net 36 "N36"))
  (pad "2" smd roundrect (at 0.5 0) (size 0.56 0.62) (layers "F.Cu" "F.Mask" "F.Paste") (roundrect_rratio 0.25) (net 2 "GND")))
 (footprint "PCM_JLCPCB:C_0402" (layer "F.Cu") (at 52.5 47)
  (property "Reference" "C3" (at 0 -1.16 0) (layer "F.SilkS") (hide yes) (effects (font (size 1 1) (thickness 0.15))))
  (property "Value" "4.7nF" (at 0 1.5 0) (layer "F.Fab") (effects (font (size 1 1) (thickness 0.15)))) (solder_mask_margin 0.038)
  (pad "1" smd roundrect (at -0.5 0) (size 0.56 0.62) (layers "F.Cu" "F.Mask" "F.Paste") (roundrect_rratio 0.25) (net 33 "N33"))
  (pad "2" smd roundrect (at 0.5 0) (size 0.56 0.62) (layers "F.Cu" "F.Mask" "F.Paste") (roundrect_rratio 0.25) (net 36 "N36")))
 (gr_rect (start 27.5 20.5) (end 57 51) (stroke (width 0.05) (type default)) (fill no) (layer "Edge.Cuts"))
 (segment (start 50 42.5) (end 50 45) (width 0.2) (layer "F.Cu") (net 34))
 (segment (start 46.5 41) (end 48.5 41) (width 0.2) (layer "F.Cu") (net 34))
 (segment (start 50 45) (end 49.13 45.87) (width 0.2) (layer "F.Cu") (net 34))
 (segment (start 49.13 45.87) (end 48.22 45.87) (width 0.2) (layer "F.Cu") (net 34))
 (segment (start 48.5 41) (end 50 42.5) (width 0.2) (layer "F.Cu") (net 34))
 (segment (start 45.889 41.611) (end 46.5 41) (width 0.2) (layer "F.Cu") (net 34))
 (segment (start 43.78 41.5) (end 43.891 41.611) (width 0.2) (layer "F.Cu") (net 34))
 (segment (start 43.391 41.611) (end 45.889 41.611) (width 0.2) (layer "F.Cu") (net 34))
 (segment (start 48.22 43) (end 48.22 44.59) (width 0.2) (layer "F.Cu") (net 35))
 (segment (start 46.5 42.5) (end 47.72 42.5) (width 0.2) (layer "F.Cu") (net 35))
 (segment (start 47.72 42.5) (end 48.22 43) (width 0.2) (layer "F.Cu") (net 35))
 (segment (start 54.5 47) (end 53 47) (width 0.2) (layer "F.Cu") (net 36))
 (segment (start 51.87 47.13) (end 52 47) (width 0.2) (layer "F.Cu") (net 33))
 (segment (start 52 47) (end 48.35 47) (width 0.2) (layer "F.Cu") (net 33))
 (segment (start 48.35 47) (end 48.22 47.13) (width 0.2) (layer "F.Cu") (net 33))
 (segment (start 41.09 44.59) (end 42.78 44.59) (width 0.2) (layer "F.Cu") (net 31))
 (segment (start 41.5 39.5) (end 40.5 40.5) (width 0.2) (layer "F.Cu") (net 31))
 (segment (start 40.5 40.5) (end 40.5 44) (width 0.2) (layer "F.Cu") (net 31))
 (segment (start 45.5 39.5) (end 41.5 39.5) (width 0.2) (layer "F.Cu") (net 31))
 (segment (start 40.5 44) (end 41.09 44.59) (width 0.2) (layer "F.Cu") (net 31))
 (segment (start 41.63 47.13) (end 41 46.5) (width 0.2) (layer "F.Cu") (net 3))
 (segment (start 41.889 40.111) (end 45.889 40.111) (width 0.2) (layer "F.Cu") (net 3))
 (segment (start 42.78 47.13) (end 41.63 47.13) (width 0.2) (layer "F.Cu") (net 3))
 (segment (start 41.1 40.9) (end 41.1 43.5) (width 0.2) (layer "F.Cu") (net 3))
 (segment (start 41.889 40.111) (end 41.1 40.9) (width 0.2) (layer "F.Cu") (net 3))
 (segment (start 50.75 39.5) (end 46.5 39.5) (width 0.2) (layer "F.Cu") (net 3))
 (segment (start 52.5 37.75) (end 50.75 39.5) (width 0.2) (layer "F.Cu") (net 3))
 (segment (start 45.889 40.111) (end 46.5 39.5) (width 0.2) (layer "F.Cu") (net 3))
 (via (at 41 46.5) (size 0.6) (drill 0.3) (layers "F.Cu" "B.Cu") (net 3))
 (via (at 41.1 43.5) (size 0.6) (drill 0.3) (layers "F.Cu" "B.Cu") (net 3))
 (segment (start 41.1 43.5) (end 41.1 46.4) (width 0.2) (layer "B.Cu") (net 3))
 (segment (start 41.1 46.4) (end 41 46.5) (width 0.2) (layer "B.Cu") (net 3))
 (segment (start 43.0671 39) (end 45.28355 36.78355) (width 0.2) (layer "F.Cu") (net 10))
 (segment (start 37 23.6) (end 37 22.4) (width 0.2) (layer "F.Cu") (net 10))
 (segment (start 38.5 24) (end 37.4 24) (width 0.2) (layer "F.Cu") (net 10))
 (segment (start 37.4 24) (end 37 23.6) (width 0.2) (layer "F.Cu") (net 10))
 (segment (start 32.5 39) (end 43.0671 39) (width 0.2) (layer "F.Cu") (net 10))
 (via (at 38.5 24) (size 0.6) (drill 0.3) (layers "F.Cu" "B.Cu") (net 10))
 (via (at 45.28355 36.78355) (size 0.6) (drill 0.3) (layers "F.Cu" "B.Cu") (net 10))
 (segment (start 45.941523 27.441523) (end 43 24.5) (width 0.2) (layer "B.Cu") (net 10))
 (segment (start 39 24.5) (end 38.5 24) (width 0.2) (layer "B.Cu") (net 10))
 (segment (start 43 24.5) (end 39 24.5) (width 0.2) (layer "B.Cu") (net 10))
 (segment (start 45.28355 36.78355) (end 45.941523 36.125577) (width 0.2) (layer "B.Cu") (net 10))
 (segment (start 45.941523 36.125577) (end 45.941523 27.441523) (width 0.2) (layer "B.Cu") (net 10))
 (segment (start 32.5 38.5) (end 42.5 38.5) (width 0.2) (layer "F.Cu") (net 11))
 (segment (start 37.5 25) (end 36 23.5) (width 0.2) (layer "F.Cu") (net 11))
 (segment (start 42.5 38.5) (end 44 37) (width 0.2) (layer "F.Cu") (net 11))
 (segment (start 44 37) (end 44 33.5) (width 0.2) (layer "F.Cu") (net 11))
 (segment (start 36 23.5) (end 36 22.4) (width 0.2) (layer "F.Cu") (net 11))
 (via (at 44 33.5) (size 0.6) (drill 0.3) (layers "F.Cu" "B.Cu") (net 11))
 (via (at 37.5 25) (size 0.6) (drill 0.3) (layers "F.Cu" "B.Cu") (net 11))
 (segment (start 44 33.5) (end 44 26.5671) (width 0.2) (layer "B.Cu") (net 11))
 (segment (start 44 26.5671) (end 42.4329 25) (width 0.2) (layer "B.Cu") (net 11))
 (segment (start 42.4329 25) (end 37.5 25) (width 0.2) (layer "B.Cu") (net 11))
 (segment (start 32.5 40) (end 34.988068 40) (width 0.2) (layer "F.Cu") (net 9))
 (segment (start 36 33) (end 34 31) (width 0.2) (layer "F.Cu") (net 9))
 (segment (start 34 31) (end 34 29.6) (width 0.2) (layer "F.Cu") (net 9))
 (segment (start 34.988068 40) (end 35.247017 39.741051) (width 0.2) (layer "F.Cu") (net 9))
 (via (at 36 33) (size 0.6) (drill 0.3) (layers "F.Cu" "B.Cu") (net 9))
 (via (at 35.247017 39.741051) (size 0.6) (drill 0.3) (layers "F.Cu" "B.Cu") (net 9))
 (segment (start 35.247017 39.741051) (end 35.258949 39.741051) (width 0.2) (layer "B.Cu") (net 9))
 (segment (start 37 38) (end 37 34) (width 0.2) (layer "B.Cu") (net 9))
 (segment (start 35.258949 39.741051) (end 37 38) (width 0.2) (layer "B.Cu") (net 9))
 (segment (start 37 34) (end 36 33) (width 0.2) (layer "B.Cu") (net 9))
 (segment (start 32.5 41.5) (end 36.131374 41.5) (width 0.2) (layer "F.Cu") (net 7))
 (segment (start 38 32) (end 37 31) (width 0.2) (layer "F.Cu") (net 7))
 (segment (start 37 31) (end 37 29.6) (width 0.2) (layer "F.Cu") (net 7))
 (segment (start 36.131374 41.5) (end 36.565687 41.065687) (width 0.2) (layer "F.Cu") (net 7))
 (via (at 36.565687 41.065687) (size 0.6) (drill 0.3) (layers "F.Cu" "B.Cu") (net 7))
 (via (at 38 32) (size 0.6) (drill 0.3) (layers "F.Cu" "B.Cu") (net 7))
 (segment (start 39 33) (end 39 38.631374) (width 0.2) (layer "B.Cu") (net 7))
 (segment (start 38 32) (end 39 33) (width 0.2) (layer "B.Cu") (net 7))
 (segment (start 39 38.631374) (end 36.565687 41.065687) (width 0.2) (layer "B.Cu") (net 7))
 (segment (start 36.762748 42) (end 37.131374 41.631374) (width 0.2) (layer "F.Cu") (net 6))
 (segment (start 32.5 42) (end 36.762748 42) (width 0.2) (layer "F.Cu") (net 6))
 (segment (start 39 31.5) (end 38 30.5) (width 0.2) (layer "F.Cu") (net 6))
 (segment (start 38 30.5) (end 38 29.6) (width 0.2) (layer "F.Cu") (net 6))
 (via (at 37.131374 41.631374) (size 0.6) (drill 0.3) (layers "F.Cu" "B.Cu") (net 6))
 (via (at 39 31.5) (size 0.6) (drill 0.3) (layers "F.Cu" "B.Cu") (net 6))
 (segment (start 40 32.5) (end 40 38.762748) (width 0.2) (layer "B.Cu") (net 6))
 (segment (start 40 32.5) (end 39 31.5) (width 0.2) (layer "B.Cu") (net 6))
 (segment (start 40 38.762748) (end 37.131374 41.631374) (width 0.2) (layer "B.Cu") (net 6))
 (segment (start 42 33) (end 42 29.6) (width 0.2) (layer "F.Cu") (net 15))
 (segment (start 39 36) (end 42 33) (width 0.2) (layer "F.Cu") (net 15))
 (segment (start 32.5 36) (end 39 36) (width 0.2) (layer "F.Cu") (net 15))
 (segment (start 37 32.5) (end 35 30.5) (width 0.2) (layer "F.Cu") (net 8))
 (segment (start 35 30.5) (end 35 29.6) (width 0.2) (layer "F.Cu") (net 8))
 (segment (start 36 40.5) (end 32.5 40.5) (width 0.2) (layer "F.Cu") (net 8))
 (via (at 37 32.5) (size 0.6) (drill 0.3) (layers "F.Cu" "B.Cu") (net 8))
 (via (at 36 40.5) (size 0.6) (drill 0.3) (layers "F.Cu" "B.Cu") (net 8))
 (segment (start 38 33.5) (end 37 32.5) (width 0.2) (layer "B.Cu") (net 8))
 (segment (start 38 38.501215) (end 38 33.5) (width 0.2) (layer "B.Cu") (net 8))
 (segment (start 36.001215 40.5) (end 38 38.501215) (width 0.2) (layer "B.Cu") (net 8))
 (segment (start 36 40.5) (end 36.001215 40.5) (width 0.2) (layer "B.Cu") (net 8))
 (segment (start 45 28) (end 45 25.5) (width 0.2) (layer "F.Cu") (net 14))
 (segment (start 39 23) (end 39 22.4) (width 0.2) (layer "F.Cu") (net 14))
 (segment (start 32.5 36.5) (end 34.5 36.5) (width 0.2) (layer "F.Cu") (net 14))
 (segment (start 40 24) (end 39 23) (width 0.2) (layer "F.Cu") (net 14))
 (segment (start 45 25.5) (end 43.5 24) (width 0.2) (layer "F.Cu") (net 14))
 (segment (start 34.5 36.5) (end 40 36.5) (width 0.2) (layer "F.Cu") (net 14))
 (segment (start 43.5 24) (end 40 24) (width 0.2) (layer "F.Cu") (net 14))
 (segment (start 40 36.5) (end 41.399 36.5) (width 0.2) (layer "F.Cu") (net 14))
 (via (at 41.399 36.5) (size 0.6) (drill 0.3) (layers "F.Cu" "B.Cu") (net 14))
 (via (at 45 28) (size 0.6) (drill 0.3) (layers "F.Cu" "B.Cu") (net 14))
 (segment (start 45 28) (end 45 34.5) (width 0.2) (layer "B.Cu") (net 14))
 (segment (start 45 34.5) (end 43 36.5) (width 0.2) (layer "B.Cu") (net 14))
 (segment (start 43 36.5) (end 41.399 36.5) (width 0.2) (layer "B.Cu") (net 14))
 (segment (start 54.5 49.5) (end 55.5 48.5) (width 0.2) (layer "F.Cu") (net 32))
 (segment (start 52 48.5) (end 53 49.5) (width 0.2) (layer "F.Cu") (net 32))
 (segment (start 51.9 48.4) (end 52 48.5) (width 0.2) (layer "F.Cu") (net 32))
 (segment (start 48.22 48.4) (end 51.9 48.4) (width 0.2) (layer "F.Cu") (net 32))
 (segment (start 53 49.5) (end 54.5 49.5) (width 0.2) (layer "F.Cu") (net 32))
 (segment (start 38.5 46) (end 38.5 47.5) (width 0.2) (layer "F.Cu") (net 1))
 (segment (start 54.98 41.5) (end 54.98 44.5) (width 0.2) (layer "F.Cu") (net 30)))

